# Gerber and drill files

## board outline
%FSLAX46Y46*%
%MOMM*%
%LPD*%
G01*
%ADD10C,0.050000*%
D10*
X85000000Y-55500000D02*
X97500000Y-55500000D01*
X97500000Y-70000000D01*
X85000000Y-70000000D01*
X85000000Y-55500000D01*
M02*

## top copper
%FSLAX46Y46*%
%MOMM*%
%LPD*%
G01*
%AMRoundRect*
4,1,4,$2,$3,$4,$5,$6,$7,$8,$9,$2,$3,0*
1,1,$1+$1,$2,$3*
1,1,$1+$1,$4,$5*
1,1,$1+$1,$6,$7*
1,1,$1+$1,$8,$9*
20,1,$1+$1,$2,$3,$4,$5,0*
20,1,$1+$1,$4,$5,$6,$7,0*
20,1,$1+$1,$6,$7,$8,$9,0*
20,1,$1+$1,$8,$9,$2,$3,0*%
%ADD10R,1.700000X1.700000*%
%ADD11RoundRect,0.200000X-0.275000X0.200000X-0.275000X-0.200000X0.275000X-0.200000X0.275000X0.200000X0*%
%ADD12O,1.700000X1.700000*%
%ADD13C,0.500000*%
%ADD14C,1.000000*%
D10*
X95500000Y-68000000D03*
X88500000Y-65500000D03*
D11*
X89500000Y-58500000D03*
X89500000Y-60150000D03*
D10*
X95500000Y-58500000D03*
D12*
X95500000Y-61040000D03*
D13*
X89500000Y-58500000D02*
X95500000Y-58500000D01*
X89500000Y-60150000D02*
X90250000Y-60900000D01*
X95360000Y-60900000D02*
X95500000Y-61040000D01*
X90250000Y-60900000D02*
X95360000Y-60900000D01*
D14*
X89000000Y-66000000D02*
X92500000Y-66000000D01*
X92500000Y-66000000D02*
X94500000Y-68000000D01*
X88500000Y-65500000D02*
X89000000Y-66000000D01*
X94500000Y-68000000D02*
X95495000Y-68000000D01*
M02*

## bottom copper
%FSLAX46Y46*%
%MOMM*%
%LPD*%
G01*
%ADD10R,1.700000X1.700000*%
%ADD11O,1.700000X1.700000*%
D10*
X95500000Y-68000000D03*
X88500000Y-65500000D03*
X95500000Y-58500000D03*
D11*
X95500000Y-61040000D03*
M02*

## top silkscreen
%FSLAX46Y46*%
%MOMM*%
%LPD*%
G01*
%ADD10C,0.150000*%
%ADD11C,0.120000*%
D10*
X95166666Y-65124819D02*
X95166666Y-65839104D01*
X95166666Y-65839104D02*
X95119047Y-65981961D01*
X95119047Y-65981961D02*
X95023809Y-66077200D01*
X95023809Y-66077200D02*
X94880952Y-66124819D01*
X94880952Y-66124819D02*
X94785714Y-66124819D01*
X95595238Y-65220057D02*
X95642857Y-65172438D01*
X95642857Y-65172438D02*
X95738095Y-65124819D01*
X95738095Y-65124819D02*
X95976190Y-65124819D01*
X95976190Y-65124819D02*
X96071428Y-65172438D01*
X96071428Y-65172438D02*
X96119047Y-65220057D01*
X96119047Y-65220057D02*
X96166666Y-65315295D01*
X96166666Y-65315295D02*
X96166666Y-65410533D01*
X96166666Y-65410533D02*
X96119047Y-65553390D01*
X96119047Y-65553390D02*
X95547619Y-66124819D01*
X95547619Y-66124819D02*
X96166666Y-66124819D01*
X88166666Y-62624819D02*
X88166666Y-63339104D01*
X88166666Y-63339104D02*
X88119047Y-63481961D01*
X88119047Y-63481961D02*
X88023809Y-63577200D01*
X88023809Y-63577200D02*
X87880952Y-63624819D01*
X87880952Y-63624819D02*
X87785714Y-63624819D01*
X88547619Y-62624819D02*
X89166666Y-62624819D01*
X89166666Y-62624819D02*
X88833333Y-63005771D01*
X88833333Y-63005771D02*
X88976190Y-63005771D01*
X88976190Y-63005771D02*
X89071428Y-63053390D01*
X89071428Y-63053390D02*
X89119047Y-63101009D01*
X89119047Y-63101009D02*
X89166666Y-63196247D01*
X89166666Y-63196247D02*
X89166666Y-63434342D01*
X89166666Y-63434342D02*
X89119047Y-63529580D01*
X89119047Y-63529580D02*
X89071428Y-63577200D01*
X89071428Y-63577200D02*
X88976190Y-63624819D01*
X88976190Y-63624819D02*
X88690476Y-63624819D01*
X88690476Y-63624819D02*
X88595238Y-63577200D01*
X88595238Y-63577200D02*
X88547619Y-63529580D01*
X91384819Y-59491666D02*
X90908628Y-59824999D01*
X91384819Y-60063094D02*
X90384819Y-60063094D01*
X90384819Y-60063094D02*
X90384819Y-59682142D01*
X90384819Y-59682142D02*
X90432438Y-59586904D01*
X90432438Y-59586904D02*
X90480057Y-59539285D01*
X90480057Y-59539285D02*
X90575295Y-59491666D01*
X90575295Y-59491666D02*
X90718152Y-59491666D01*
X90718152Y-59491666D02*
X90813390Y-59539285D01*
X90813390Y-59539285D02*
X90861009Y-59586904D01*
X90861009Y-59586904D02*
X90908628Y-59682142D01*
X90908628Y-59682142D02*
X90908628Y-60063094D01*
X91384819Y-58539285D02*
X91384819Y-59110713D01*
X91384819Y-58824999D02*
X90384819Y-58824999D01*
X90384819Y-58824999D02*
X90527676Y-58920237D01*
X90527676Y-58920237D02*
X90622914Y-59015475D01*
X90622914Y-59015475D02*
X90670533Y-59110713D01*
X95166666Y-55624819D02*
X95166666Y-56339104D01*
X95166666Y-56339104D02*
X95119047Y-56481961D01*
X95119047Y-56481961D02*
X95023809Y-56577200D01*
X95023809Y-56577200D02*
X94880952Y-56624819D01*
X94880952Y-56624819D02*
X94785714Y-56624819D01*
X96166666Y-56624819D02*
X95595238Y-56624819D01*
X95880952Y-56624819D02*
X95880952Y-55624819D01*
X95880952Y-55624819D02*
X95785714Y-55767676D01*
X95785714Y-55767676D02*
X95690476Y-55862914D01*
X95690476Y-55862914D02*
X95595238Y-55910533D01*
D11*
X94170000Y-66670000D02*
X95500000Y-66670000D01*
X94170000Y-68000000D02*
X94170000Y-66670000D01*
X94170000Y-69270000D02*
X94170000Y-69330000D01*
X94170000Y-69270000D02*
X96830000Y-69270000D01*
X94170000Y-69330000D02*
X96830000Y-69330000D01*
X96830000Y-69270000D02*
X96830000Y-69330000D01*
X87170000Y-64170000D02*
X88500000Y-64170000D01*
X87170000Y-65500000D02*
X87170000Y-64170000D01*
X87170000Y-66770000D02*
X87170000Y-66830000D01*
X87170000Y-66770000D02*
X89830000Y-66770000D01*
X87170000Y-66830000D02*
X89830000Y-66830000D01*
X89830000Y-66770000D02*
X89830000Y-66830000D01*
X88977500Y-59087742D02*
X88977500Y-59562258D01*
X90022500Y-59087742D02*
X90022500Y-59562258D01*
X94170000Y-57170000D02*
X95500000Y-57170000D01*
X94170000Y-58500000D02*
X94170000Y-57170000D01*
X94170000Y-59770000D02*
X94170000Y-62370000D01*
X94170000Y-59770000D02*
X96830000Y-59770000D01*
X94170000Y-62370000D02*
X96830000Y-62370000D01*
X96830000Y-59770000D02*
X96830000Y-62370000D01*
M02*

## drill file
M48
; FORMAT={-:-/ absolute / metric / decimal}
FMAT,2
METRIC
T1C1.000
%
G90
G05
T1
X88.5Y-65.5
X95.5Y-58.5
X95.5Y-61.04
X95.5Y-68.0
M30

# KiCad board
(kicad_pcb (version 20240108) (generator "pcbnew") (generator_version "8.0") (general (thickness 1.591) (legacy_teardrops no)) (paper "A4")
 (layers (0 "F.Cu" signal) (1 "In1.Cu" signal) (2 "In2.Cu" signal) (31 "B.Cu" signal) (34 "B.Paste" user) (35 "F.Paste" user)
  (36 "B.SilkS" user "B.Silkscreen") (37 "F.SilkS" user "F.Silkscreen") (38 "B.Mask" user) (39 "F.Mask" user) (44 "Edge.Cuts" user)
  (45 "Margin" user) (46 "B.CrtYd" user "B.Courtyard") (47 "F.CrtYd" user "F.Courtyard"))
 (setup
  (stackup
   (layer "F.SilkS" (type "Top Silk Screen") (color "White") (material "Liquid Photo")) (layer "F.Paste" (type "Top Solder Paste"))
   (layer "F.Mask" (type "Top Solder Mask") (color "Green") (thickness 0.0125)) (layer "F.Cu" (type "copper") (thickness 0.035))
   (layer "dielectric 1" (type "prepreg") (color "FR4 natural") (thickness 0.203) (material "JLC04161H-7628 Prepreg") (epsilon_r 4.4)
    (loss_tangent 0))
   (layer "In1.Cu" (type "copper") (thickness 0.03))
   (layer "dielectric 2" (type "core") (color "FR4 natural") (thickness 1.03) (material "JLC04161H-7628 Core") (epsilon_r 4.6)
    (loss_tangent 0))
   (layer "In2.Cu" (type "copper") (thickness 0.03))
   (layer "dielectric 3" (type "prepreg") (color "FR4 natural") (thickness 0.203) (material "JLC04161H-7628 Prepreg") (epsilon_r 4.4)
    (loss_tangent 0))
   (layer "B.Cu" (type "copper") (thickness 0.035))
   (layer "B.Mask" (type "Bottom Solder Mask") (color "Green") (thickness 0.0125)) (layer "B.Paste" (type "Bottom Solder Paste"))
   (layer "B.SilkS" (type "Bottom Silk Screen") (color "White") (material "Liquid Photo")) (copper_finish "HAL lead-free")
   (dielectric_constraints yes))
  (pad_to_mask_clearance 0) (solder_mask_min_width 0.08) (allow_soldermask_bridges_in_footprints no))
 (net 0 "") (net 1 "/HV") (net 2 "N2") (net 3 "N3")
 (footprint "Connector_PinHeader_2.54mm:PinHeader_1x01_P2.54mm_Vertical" (layer "F.Cu") (at 95.5 68)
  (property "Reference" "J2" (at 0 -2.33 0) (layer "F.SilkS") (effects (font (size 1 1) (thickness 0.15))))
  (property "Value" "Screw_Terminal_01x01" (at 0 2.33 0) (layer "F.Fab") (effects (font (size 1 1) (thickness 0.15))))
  (fp_line (start -1.33 -1.33) (end 0 -1.33) (stroke (width 0.12) (type solid)) (layer "F.SilkS"))
  (fp_line (start -1.33 0) (end -1.33 -1.33) (stroke (width 0.12) (type solid)) (layer "F.SilkS"))
  (fp_line (start -1.33 1.27) (end -1.33 1.33) (stroke (width 0.12) (type solid)) (layer "F.SilkS"))
  (fp_line (start -1.33 1.27) (end 1.33 1.27) (stroke (width 0.12) (type solid)) (layer "F.SilkS"))
  (fp_line (start -1.33 1.33) (end 1.33 1.33) (stroke (width 0.12) (type solid)) (layer "F.SilkS"))
  (fp_line (start 1.33 1.27) (end 1.33 1.33) (stroke (width 0.12) (type solid)) (layer "F.SilkS"))
  (pad "1" thru_hole rect (at 0 0) (size 1.7 1.7) (drill 1) (layers "*.Cu" "*.Mask") (remove_unused_layers no) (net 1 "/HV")))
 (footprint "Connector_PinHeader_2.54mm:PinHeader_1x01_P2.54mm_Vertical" (layer "F.Cu") (at 88.5 65.5)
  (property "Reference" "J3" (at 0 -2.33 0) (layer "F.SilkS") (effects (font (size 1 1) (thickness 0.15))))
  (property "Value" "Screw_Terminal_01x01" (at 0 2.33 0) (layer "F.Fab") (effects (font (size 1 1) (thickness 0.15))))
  (fp_line (start -1.33 -1.33) (end 0 -1.33) (stroke (width 0.12) (type solid)) (layer "F.SilkS"))
  (fp_line (start -1.33 0) (end -1.33 -1.33) (stroke (width 0.12) (type solid)) (layer "F.SilkS"))
  (fp_line (start -1.33 1.27) (end -1.33 1.33) (stroke (width 0.12) (type solid)) (layer "F.SilkS"))
  (fp_line (start -1.33 1.27) (end 1.33 1.27) (stroke (width 0.12) (type solid)) (layer "F.SilkS"))
  (fp_line (start -1.33 1.33) (end 1.33 1.33) (stroke (width 0.12) (type solid)) (layer "F.SilkS"))
  (fp_line (start 1.33 1.27) (end 1.33 1.33) (stroke (width 0.12) (type solid)) (layer "F.SilkS"))
  (pad "1" thru_hole rect (at 0 0) (size 1.7 1.7) (drill 1) (layers "*.Cu" "*.Mask") (remove_unused_layers no) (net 1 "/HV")))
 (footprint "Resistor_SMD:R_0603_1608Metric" (layer "F.Cu") (at 89.5 59.325 -90)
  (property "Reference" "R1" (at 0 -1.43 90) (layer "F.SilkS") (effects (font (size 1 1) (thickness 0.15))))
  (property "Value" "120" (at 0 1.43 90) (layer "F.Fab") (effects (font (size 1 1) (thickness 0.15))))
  (fp_line (start -0.237258 0.5225) (end 0.237258 0.5225) (stroke (width 0.12) (type solid)) (layer "F.SilkS"))
  (fp_line (start -0.237258 -0.5225) (end 0.237258 -0.5225) (stroke (width 0.12) (type solid)) (layer "F.SilkS"))
  (pad "1" smd roundrect (at -0.825 0 270) (size 0.8 0.95) (layers "F.Cu" "F.Paste" "F.Mask") (roundrect_rratio 0.25) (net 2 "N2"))
  (pad "2" smd roundrect (at 0.825 0 270) (size 0.8 0.95) (layers "F.Cu" "F.Paste" "F.Mask") (roundrect_rratio 0.25) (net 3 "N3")))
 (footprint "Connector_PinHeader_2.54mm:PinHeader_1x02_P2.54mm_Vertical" (layer "F.Cu") (at 95.5 58.5)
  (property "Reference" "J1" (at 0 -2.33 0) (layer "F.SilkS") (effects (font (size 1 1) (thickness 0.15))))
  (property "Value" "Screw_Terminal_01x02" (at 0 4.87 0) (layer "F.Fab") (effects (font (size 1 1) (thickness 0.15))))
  (fp_line (start -1.33 -1.33) (end 0 -1.33) (stroke (width 0.12) (type solid)) (layer "F.SilkS"))
  (fp_line (start -1.33 0) (end -1.33 -1.33) (stroke (width 0.12) (type solid)) (layer "F.SilkS"))
  (fp_line (start -1.33 1.27) (end -1.33 3.87) (stroke (width 0.12) (type solid)) (layer "F.SilkS"))
  (fp_line (start -1.33 1.27) (end 1.33 1.27) (stroke (width 0.12) (type solid)) (layer "F.SilkS"))
  (fp_line (start -1.33 3.87) (end 1.33 3.87) (stroke (width 0.12) (type solid)) (layer "F.SilkS"))
  (fp_line (start 1.33 1.27) (end 1.33 3.87) (stroke (width 0.12) (type solid)) (layer "F.SilkS"))
  (pad "1" thru_hole rect (at 0 0) (size 1.7 1.7) (drill 1) (layers "*.Cu" "*.Mask") (remove_unused_layers no) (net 2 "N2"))
  (pad "2" thru_hole oval (at 0 2.54) (size 1.7 1.7) (drill 1) (layers "*.Cu" "*.Mask") (remove_unused_layers no) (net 3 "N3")))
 (gr_rect (start 85 55.5) (end 97.5 70) (stroke (width 0.05) (type default)) (fill none) (layer "Edge.Cuts"))
 (segment (start 89.5 58.5) (end 95.5 58.5) (width 0.5) (layer "F.Cu") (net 2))
 (segment (start 89.5 60.15) (end 90.25 60.9) (width 0.5) (layer "F.Cu") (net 3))
 (segment (start 95.36 60.9) (end 95.5 61.04) (width 0.5) (layer "F.Cu") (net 3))
 (segment (start 90.25 60.9) (end 95.36 60.9) (width 0.5) (layer "F.Cu") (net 3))
 (segment (start 89 66) (end 92.5 66) (width 1) (layer "F.Cu") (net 1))
 (segment (start 92.5 66) (end 94.5 68) (width 1) (layer "F.Cu") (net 1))
 (segment (start 88.5 65.5) (end 89 66) (width 1) (layer "F.Cu") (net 1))
 (segment (start 94.5 68) (end 95.495 68) (width 1) (layer "F.Cu") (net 1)))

